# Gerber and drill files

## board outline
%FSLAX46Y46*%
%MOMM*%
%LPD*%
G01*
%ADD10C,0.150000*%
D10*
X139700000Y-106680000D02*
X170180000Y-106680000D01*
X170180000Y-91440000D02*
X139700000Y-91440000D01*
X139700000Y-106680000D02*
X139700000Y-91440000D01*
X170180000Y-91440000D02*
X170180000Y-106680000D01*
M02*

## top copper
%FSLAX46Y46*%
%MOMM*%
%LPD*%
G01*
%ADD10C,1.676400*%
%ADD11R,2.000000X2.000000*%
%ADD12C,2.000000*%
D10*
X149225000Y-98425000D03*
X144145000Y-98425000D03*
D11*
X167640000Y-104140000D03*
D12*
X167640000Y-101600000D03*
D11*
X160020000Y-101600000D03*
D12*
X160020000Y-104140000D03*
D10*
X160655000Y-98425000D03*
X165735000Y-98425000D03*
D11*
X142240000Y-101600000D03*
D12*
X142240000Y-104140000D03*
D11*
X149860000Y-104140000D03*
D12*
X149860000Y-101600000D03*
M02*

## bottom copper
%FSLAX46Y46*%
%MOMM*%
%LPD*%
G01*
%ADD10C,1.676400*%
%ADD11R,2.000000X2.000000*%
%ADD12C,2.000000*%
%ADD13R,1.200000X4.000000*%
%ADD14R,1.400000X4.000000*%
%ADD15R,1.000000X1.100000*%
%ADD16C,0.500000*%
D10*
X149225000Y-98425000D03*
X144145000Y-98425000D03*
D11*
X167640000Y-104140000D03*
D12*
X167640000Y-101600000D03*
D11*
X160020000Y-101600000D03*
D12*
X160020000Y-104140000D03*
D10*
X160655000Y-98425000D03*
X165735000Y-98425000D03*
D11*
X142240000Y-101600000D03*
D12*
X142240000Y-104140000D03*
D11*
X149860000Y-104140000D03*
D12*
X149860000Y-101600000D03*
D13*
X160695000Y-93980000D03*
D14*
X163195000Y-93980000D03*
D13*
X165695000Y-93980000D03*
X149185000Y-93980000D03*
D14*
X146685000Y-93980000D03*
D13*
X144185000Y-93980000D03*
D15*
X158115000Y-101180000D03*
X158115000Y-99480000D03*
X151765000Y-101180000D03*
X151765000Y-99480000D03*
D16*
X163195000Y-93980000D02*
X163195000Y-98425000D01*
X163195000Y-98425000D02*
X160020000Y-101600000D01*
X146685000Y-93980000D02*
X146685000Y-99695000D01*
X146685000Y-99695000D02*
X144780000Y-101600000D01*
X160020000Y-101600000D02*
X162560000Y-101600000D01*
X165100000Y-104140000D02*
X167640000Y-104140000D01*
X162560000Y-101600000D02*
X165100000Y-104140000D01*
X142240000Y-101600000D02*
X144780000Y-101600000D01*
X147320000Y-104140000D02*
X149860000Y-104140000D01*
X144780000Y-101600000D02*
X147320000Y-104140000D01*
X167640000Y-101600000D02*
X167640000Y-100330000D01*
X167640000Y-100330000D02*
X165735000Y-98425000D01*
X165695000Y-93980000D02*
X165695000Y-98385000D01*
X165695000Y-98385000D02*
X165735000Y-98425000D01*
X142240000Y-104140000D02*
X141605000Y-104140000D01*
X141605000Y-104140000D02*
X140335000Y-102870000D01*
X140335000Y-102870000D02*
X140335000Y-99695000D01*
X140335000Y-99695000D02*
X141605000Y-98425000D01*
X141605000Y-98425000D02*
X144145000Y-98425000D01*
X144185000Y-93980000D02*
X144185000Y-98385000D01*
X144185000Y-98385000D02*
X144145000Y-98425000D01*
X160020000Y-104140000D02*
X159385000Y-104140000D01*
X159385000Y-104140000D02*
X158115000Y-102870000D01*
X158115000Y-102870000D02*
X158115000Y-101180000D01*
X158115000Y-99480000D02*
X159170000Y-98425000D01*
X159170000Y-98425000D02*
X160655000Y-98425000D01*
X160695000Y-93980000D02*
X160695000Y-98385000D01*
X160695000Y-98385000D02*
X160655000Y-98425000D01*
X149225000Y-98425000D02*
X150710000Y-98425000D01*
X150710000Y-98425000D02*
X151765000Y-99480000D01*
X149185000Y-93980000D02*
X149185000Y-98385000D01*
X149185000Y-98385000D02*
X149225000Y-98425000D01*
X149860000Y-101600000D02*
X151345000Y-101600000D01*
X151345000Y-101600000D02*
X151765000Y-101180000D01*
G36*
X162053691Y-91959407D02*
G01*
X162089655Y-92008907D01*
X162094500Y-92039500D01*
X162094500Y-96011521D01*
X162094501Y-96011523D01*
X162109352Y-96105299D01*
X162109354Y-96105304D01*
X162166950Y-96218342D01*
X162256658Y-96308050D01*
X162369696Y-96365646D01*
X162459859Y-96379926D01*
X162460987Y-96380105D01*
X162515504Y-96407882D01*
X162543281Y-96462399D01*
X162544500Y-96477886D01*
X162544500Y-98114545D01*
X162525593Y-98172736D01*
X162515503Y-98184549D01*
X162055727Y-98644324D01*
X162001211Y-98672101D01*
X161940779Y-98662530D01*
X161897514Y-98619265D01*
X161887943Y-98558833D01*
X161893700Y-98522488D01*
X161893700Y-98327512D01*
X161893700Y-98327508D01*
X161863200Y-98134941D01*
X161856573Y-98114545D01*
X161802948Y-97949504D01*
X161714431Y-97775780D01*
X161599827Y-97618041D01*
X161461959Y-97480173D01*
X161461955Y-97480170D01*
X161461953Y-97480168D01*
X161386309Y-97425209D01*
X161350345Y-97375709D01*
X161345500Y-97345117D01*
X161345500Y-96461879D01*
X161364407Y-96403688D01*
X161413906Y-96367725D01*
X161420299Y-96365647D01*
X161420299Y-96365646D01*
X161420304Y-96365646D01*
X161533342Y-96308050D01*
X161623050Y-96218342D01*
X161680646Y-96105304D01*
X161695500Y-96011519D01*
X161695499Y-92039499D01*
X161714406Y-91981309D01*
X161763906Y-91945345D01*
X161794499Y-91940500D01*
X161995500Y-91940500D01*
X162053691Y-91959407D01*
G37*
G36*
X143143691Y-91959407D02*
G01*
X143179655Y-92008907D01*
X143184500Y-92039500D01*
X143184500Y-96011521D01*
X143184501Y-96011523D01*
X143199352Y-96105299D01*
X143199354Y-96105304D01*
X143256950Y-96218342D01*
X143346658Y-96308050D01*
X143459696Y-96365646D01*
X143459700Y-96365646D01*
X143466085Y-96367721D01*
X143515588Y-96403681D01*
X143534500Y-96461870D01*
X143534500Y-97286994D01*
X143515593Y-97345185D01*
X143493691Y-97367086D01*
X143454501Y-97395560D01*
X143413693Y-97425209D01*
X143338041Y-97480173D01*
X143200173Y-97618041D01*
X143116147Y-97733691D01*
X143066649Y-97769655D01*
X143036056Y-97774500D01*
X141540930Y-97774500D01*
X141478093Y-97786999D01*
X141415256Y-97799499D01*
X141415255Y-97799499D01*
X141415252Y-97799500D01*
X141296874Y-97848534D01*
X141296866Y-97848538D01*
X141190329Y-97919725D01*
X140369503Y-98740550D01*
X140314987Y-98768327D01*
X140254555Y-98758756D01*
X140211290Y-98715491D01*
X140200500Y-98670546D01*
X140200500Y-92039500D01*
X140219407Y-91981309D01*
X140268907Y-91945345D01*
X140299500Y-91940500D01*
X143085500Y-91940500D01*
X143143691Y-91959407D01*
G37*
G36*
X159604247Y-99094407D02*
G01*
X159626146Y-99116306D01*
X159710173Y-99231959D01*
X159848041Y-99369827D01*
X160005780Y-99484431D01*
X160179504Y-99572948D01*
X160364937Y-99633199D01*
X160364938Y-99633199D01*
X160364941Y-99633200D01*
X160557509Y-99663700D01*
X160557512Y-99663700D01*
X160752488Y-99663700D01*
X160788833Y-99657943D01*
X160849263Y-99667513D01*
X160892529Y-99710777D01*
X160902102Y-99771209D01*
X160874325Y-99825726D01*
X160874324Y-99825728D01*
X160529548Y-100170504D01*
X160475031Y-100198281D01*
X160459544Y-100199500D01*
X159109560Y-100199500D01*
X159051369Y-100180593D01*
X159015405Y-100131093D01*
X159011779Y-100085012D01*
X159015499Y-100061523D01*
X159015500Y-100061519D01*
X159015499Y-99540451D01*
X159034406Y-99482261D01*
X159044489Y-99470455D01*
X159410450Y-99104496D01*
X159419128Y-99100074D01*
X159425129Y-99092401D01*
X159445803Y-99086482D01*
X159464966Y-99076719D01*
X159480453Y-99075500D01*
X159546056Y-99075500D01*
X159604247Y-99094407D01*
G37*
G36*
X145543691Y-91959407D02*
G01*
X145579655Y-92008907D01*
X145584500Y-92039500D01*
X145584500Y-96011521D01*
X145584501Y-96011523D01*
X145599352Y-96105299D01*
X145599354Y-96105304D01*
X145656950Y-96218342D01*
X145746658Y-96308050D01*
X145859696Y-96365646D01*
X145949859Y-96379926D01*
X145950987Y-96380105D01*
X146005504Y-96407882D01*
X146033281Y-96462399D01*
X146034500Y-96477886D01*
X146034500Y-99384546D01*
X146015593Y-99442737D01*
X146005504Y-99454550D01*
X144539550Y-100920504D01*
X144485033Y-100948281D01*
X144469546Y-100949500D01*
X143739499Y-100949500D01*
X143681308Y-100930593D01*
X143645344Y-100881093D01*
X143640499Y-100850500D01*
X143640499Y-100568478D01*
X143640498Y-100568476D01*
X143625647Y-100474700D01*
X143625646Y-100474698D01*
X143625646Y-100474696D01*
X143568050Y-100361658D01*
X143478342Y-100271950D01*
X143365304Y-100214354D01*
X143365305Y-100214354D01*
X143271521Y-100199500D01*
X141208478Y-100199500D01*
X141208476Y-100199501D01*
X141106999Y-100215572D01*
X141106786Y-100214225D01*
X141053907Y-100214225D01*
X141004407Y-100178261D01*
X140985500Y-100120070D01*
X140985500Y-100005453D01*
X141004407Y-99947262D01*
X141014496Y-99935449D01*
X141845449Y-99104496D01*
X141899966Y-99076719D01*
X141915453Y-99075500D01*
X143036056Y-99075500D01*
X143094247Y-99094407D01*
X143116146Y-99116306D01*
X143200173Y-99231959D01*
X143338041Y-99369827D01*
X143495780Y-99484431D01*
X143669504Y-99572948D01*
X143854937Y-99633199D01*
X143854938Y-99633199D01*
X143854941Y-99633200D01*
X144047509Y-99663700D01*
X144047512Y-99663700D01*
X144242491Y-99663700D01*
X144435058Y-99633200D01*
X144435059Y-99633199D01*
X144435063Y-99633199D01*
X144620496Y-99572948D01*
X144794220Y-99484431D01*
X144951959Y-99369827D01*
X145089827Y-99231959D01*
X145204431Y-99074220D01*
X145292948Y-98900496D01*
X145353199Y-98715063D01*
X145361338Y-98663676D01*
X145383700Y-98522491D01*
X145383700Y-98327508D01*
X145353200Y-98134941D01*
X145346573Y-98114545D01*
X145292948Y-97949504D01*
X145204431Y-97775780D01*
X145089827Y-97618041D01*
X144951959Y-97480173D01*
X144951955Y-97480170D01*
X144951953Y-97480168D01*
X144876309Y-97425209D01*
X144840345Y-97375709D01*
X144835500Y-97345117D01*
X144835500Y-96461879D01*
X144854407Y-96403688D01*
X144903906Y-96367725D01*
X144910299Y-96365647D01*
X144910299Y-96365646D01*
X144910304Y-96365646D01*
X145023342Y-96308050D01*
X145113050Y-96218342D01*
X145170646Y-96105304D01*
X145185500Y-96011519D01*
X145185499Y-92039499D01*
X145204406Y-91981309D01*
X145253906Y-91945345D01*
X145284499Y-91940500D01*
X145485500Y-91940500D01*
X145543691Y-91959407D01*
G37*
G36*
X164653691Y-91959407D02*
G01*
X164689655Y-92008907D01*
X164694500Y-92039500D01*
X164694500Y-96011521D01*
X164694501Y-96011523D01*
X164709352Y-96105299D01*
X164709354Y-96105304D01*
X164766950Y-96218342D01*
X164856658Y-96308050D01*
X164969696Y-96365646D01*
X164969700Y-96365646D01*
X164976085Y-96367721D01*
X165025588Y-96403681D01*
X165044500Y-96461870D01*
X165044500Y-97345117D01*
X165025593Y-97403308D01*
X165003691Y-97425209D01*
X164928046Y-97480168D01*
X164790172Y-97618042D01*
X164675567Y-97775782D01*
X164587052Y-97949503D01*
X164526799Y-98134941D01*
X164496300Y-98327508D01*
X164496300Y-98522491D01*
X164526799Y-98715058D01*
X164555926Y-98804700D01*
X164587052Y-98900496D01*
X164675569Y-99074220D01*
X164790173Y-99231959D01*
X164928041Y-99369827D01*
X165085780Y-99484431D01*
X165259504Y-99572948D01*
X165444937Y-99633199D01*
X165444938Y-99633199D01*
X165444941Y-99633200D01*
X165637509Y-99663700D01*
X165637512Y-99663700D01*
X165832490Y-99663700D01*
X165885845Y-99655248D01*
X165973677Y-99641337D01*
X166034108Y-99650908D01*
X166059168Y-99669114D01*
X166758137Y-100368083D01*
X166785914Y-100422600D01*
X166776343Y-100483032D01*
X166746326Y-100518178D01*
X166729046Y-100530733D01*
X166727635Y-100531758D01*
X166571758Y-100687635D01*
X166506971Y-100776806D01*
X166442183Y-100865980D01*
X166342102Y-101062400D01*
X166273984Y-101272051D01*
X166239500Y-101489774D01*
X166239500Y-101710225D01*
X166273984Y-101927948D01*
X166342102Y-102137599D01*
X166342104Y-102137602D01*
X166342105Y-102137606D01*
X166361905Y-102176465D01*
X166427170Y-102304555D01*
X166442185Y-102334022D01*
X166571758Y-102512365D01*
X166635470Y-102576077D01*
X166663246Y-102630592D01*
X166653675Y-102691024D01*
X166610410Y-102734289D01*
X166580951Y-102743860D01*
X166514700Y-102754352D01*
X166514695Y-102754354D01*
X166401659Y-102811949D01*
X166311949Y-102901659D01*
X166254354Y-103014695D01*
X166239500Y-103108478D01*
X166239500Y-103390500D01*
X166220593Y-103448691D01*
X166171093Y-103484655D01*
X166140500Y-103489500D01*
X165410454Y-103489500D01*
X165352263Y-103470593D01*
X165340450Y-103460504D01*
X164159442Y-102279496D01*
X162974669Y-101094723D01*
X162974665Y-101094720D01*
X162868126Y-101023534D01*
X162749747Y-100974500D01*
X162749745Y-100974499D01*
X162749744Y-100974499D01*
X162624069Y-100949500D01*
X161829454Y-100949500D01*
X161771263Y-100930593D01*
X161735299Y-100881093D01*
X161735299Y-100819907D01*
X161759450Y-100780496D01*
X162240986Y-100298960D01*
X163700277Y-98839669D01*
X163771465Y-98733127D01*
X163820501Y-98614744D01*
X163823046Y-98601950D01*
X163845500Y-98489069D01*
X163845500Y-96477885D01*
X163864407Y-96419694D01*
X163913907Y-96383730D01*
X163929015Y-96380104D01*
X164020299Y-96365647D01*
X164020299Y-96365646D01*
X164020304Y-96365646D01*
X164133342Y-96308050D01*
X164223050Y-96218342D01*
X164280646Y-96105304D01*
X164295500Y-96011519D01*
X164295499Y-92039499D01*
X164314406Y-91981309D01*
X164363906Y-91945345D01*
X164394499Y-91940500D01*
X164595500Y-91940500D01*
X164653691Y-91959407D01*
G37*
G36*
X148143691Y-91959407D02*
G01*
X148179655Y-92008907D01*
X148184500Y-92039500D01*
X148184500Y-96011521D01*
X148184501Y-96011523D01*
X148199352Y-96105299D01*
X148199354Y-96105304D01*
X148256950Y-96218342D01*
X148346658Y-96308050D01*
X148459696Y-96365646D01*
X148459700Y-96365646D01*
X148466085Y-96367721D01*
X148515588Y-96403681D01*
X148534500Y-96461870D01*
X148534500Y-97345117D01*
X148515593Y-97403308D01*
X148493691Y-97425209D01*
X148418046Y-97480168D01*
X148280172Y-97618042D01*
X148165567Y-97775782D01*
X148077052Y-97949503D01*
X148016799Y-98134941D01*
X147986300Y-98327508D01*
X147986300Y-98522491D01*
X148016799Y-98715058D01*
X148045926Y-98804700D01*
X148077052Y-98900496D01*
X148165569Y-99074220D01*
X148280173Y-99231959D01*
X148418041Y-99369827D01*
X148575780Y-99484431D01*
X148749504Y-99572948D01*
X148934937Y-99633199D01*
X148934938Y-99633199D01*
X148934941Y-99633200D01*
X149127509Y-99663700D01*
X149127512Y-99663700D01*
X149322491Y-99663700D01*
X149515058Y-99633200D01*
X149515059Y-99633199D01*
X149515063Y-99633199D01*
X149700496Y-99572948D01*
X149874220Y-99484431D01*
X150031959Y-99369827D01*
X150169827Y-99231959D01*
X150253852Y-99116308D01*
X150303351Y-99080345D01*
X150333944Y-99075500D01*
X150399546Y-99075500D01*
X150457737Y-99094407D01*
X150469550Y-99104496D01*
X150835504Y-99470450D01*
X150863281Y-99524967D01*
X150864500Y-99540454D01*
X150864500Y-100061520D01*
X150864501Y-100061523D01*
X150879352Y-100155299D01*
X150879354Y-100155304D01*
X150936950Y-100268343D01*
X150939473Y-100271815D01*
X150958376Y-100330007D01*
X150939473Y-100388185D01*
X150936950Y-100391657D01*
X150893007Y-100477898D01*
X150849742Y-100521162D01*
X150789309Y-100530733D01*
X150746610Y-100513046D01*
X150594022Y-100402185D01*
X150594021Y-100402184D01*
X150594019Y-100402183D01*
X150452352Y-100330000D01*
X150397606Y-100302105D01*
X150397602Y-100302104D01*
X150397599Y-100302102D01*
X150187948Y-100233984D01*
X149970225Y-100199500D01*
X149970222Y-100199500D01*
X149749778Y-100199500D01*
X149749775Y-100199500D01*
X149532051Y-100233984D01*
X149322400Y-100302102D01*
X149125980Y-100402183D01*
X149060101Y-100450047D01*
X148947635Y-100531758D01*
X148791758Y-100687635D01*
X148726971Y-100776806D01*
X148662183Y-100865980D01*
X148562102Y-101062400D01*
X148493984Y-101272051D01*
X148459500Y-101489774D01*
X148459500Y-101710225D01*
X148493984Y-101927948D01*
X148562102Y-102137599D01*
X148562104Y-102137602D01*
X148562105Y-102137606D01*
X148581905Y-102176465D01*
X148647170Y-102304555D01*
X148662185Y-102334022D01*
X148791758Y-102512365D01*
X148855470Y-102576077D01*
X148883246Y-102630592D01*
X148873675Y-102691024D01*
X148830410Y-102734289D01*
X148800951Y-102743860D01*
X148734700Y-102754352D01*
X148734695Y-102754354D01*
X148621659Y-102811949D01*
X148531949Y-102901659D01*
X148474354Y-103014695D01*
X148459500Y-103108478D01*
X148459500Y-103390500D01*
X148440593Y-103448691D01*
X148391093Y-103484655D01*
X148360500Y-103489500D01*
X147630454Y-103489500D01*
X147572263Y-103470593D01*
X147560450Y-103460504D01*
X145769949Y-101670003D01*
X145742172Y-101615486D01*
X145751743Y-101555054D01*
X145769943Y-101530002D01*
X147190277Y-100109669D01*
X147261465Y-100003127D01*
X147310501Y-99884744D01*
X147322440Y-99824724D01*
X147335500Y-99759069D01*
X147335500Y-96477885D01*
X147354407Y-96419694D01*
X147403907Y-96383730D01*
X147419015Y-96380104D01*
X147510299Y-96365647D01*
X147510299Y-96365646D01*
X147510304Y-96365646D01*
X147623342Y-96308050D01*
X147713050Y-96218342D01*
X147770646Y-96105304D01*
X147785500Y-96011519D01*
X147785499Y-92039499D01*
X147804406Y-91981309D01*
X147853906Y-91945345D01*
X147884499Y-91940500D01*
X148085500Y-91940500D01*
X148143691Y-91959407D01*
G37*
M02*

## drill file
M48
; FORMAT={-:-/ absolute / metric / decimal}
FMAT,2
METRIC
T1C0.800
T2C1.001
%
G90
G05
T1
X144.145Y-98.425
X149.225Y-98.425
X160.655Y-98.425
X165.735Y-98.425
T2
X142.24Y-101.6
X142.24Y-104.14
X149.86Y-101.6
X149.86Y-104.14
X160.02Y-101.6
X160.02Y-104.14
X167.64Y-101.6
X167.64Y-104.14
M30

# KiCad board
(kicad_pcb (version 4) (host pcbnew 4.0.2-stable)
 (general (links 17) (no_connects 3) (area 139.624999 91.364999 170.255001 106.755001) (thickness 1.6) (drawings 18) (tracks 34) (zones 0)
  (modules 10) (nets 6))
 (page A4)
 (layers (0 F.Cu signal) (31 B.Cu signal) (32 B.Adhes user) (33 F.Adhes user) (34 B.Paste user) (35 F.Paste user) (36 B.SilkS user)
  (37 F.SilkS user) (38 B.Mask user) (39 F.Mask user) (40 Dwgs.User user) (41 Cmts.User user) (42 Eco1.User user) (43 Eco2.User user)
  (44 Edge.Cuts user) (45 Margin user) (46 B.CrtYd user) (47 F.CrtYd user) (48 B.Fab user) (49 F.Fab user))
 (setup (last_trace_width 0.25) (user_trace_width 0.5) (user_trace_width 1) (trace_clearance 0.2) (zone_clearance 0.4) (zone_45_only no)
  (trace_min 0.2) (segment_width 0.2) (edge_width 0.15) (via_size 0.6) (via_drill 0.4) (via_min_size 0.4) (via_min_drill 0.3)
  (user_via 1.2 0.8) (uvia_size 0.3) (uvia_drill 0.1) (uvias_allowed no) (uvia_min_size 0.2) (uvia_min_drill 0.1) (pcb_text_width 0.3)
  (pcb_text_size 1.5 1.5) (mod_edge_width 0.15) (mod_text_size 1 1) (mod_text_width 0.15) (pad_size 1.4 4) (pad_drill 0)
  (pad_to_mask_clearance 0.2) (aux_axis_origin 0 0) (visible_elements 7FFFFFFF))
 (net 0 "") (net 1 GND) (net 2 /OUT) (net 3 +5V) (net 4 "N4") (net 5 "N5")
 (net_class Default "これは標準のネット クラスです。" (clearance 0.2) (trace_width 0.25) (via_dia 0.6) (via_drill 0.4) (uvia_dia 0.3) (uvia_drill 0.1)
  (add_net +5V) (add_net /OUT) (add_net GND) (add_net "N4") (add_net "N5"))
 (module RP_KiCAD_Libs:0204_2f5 (layer F.Cu) (at 146.685 98.425 180)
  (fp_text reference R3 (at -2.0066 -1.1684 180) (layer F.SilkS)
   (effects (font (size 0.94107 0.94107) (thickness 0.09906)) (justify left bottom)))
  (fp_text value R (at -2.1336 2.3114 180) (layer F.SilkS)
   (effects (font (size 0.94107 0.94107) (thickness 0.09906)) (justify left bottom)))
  (pad 1 thru_hole circle (at -2.54 0 180) (size 1.6764 1.6764) (drill 0.8) (layers *.Cu *.Mask) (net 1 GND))
  (pad 2 thru_hole circle (at 2.54 0 180) (size 1.6764 1.6764) (drill 0.8) (layers *.Cu *.Mask) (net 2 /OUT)))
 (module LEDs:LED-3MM (layer F.Cu) (at 167.64 104.14 90)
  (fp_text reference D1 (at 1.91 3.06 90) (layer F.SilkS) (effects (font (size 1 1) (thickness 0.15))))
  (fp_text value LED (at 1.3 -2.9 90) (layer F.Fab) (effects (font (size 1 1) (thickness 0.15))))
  (pad 1 thru_hole rect (at 0 0 180) (size 2 2) (drill 1.00076) (layers *.Cu *.Mask F.SilkS) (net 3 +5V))
  (pad 2 thru_hole circle (at 2.54 0 90) (size 2 2) (drill 1.00076) (layers *.Cu *.Mask F.SilkS) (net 2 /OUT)))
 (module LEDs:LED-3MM (layer F.Cu) (at 160.02 101.6 270)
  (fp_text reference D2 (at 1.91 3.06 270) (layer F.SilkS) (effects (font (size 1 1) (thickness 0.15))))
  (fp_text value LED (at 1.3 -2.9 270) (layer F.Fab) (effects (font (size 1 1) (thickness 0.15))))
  (pad 1 thru_hole rect (at 0 0) (size 2 2) (drill 1.00076) (layers *.Cu *.Mask F.SilkS) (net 3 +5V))
  (pad 2 thru_hole circle (at 2.54 0 270) (size 2 2) (drill 1.00076) (layers *.Cu *.Mask F.SilkS) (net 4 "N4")))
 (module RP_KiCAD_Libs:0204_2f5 (layer F.Cu) (at 163.195 98.425)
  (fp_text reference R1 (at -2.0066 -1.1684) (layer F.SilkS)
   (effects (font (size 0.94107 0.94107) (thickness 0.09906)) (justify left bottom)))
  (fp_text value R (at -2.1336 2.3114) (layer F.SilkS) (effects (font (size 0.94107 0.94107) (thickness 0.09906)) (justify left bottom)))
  (pad 1 thru_hole circle (at -2.54 0) (size 1.6764 1.6764) (drill 0.8) (layers *.Cu *.Mask) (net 1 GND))
  (pad 2 thru_hole circle (at 2.54 0) (size 1.6764 1.6764) (drill 0.8) (layers *.Cu *.Mask) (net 2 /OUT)))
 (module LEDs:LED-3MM (layer F.Cu) (at 142.24 101.6 270)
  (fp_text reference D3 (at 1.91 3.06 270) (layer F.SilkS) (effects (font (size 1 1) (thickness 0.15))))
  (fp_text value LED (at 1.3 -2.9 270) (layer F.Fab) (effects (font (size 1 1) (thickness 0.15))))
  (pad 1 thru_hole rect (at 0 0) (size 2 2) (drill 1.00076) (layers *.Cu *.Mask F.SilkS) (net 3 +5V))
  (pad 2 thru_hole circle (at 2.54 0 270) (size 2 2) (drill 1.00076) (layers *.Cu *.Mask F.SilkS) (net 2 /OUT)))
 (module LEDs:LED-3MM (layer F.Cu) (at 149.86 104.14 90)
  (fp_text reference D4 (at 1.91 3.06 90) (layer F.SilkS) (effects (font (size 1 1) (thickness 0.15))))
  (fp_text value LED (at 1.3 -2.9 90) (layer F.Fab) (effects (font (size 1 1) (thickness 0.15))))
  (pad 1 thru_hole rect (at 0 0 180) (size 2 2) (drill 1.00076) (layers *.Cu *.Mask F.SilkS) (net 3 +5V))
  (pad 2 thru_hole circle (at 2.54 0 90) (size 2 2) (drill 1.00076) (layers *.Cu *.Mask F.SilkS) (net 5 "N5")))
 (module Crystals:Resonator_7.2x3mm (layer B.Cu) (at 163.195 93.98)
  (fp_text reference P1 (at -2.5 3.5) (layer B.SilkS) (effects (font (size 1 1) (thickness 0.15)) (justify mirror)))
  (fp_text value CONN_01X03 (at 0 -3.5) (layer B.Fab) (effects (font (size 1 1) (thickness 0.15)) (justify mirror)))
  (pad 1 smd rect (at -2.5 0) (size 1.2 4) (layers B.Cu B.Paste B.Mask) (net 1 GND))
  (pad 2 smd rect (at 0 0) (size 1.4 4) (layers B.Cu B.Paste B.Mask) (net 3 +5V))
  (pad 3 smd rect (at 2.5 0) (size 1.2 4) (layers B.Cu B.Paste B.Mask) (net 2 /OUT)))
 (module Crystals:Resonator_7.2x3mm (layer B.Cu) (at 146.685 93.98 180)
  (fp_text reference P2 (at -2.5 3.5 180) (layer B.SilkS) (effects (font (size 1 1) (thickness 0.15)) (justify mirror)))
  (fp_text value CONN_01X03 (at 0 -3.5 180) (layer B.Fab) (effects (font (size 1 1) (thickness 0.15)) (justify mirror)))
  (pad 1 smd rect (at -2.5 0 180) (size 1.2 4) (layers B.Cu B.Paste B.Mask) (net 1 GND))
  (pad 2 smd rect (at 0 0 180) (size 1.4 4) (layers B.Cu B.Paste B.Mask) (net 3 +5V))
  (pad 3 smd rect (at 2.5 0 180) (size 1.2 4) (layers B.Cu B.Paste B.Mask) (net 2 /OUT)))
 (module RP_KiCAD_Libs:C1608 (layer B.Cu) (at 158.115 100.33 90)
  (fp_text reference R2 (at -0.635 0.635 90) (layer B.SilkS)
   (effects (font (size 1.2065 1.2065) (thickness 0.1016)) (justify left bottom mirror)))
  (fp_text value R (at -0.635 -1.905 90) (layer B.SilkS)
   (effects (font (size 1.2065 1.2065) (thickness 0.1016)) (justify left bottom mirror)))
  (pad 1 smd rect (at -0.85 0 90) (size 1.1 1) (layers B.Cu B.Paste B.Mask) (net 4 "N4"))
  (pad 2 smd rect (at 0.85 0 90) (size 1.1 1) (layers B.Cu B.Paste B.Mask) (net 1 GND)))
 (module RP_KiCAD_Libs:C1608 (layer B.Cu) (at 151.765 100.33 90)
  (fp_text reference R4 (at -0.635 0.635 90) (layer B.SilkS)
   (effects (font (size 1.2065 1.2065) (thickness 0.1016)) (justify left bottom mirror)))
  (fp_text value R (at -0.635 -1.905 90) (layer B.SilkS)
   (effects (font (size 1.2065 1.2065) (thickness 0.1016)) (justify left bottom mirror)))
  (pad 1 smd rect (at -0.85 0 90) (size 1.1 1) (layers B.Cu B.Paste B.Mask) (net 5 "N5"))
  (pad 2 smd rect (at 0.85 0 90) (size 1.1 1) (layers B.Cu B.Paste B.Mask) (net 1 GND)))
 (gr_line (start 139.7 106.68) (end 170.18 106.68) (angle 90) (layer Edge.Cuts) (width 0.15))
 (gr_line (start 170.18 91.44) (end 139.7 91.44) (angle 90) (layer Edge.Cuts) (width 0.15))
 (gr_line (start 139.7 106.68) (end 139.7 91.44) (angle 90) (layer Edge.Cuts) (width 0.15))
 (gr_line (start 170.18 91.44) (end 170.18 106.68) (angle 90) (layer Edge.Cuts) (width 0.15))
 (segment (start 163.195 93.98) (end 163.195 98.425) (width 0.5) (layer B.Cu) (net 3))
 (segment (start 163.195 98.425) (end 160.02 101.6) (width 0.5) (layer B.Cu) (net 3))
 (segment (start 146.685 93.98) (end 146.685 99.695) (width 0.5) (layer B.Cu) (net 3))
 (segment (start 146.685 99.695) (end 144.78 101.6) (width 0.5) (layer B.Cu) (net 3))
 (segment (start 160.02 101.6) (end 162.56 101.6) (width 0.5) (layer B.Cu) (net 3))
 (segment (start 165.1 104.14) (end 167.64 104.14) (width 0.5) (layer B.Cu) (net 3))
 (segment (start 162.56 101.6) (end 165.1 104.14) (width 0.5) (layer B.Cu) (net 3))
 (segment (start 142.24 101.6) (end 144.78 101.6) (width 0.5) (layer B.Cu) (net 3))
 (segment (start 147.32 104.14) (end 149.86 104.14) (width 0.5) (layer B.Cu) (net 3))
 (segment (start 144.78 101.6) (end 147.32 104.14) (width 0.5) (layer B.Cu) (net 3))
 (segment (start 167.64 101.6) (end 167.64 100.33) (width 0.5) (layer B.Cu) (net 2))
 (segment (start 167.64 100.33) (end 165.735 98.425) (width 0.5) (layer B.Cu) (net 2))
 (segment (start 165.695 93.98) (end 165.695 98.385) (width 0.5) (layer B.Cu) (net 2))
 (segment (start 165.695 98.385) (end 165.735 98.425) (width 0.5) (layer B.Cu) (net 2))
 (segment (start 142.24 104.14) (end 141.605 104.14) (width 0.5) (layer B.Cu) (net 2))
 (segment (start 141.605 104.14) (end 140.335 102.87) (width 0.5) (layer B.Cu) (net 2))
 (segment (start 140.335 102.87) (end 140.335 99.695) (width 0.5) (layer B.Cu) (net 2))
 (segment (start 140.335 99.695) (end 141.605 98.425) (width 0.5) (layer B.Cu) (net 2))
 (segment (start 141.605 98.425) (end 144.145 98.425) (width 0.5) (layer B.Cu) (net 2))
 (segment (start 144.185 93.98) (end 144.185 98.385) (width 0.5) (layer B.Cu) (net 2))
 (segment (start 144.185 98.385) (end 144.145 98.425) (width 0.5) (layer B.Cu) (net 2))
 (segment (start 160.02 104.14) (end 159.385 104.14) (width 0.5) (layer B.Cu) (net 4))
 (segment (start 159.385 104.14) (end 158.115 102.87) (width 0.5) (layer B.Cu) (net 4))
 (segment (start 158.115 102.87) (end 158.115 101.18) (width 0.5) (layer B.Cu) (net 4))
 (segment (start 158.115 99.48) (end 159.17 98.425) (width 0.5) (layer B.Cu) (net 1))
 (segment (start 159.17 98.425) (end 160.655 98.425) (width 0.5) (layer B.Cu) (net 1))
 (segment (start 160.695 93.98) (end 160.695 98.385) (width 0.5) (layer B.Cu) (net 1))
 (segment (start 160.695 98.385) (end 160.655 98.425) (width 0.5) (layer B.Cu) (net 1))
 (segment (start 149.225 98.425) (end 150.71 98.425) (width 0.5) (layer B.Cu) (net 1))
 (segment (start 150.71 98.425) (end 151.765 99.48) (width 0.5) (layer B.Cu) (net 1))
 (segment (start 149.185 93.98) (end 149.185 98.385) (width 0.5) (layer B.Cu) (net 1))
 (segment (start 149.185 98.385) (end 149.225 98.425) (width 0.5) (layer B.Cu) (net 1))
 (segment (start 149.86 101.6) (end 151.345 101.6) (width 0.5) (layer B.Cu) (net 5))
 (segment (start 151.345 101.6) (end 151.765 101.18) (width 0.5) (layer B.Cu) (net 5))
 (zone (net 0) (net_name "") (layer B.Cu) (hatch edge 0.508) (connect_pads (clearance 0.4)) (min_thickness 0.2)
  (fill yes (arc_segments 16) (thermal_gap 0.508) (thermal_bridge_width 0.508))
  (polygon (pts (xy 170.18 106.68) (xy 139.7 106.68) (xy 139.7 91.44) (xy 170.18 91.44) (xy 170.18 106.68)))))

